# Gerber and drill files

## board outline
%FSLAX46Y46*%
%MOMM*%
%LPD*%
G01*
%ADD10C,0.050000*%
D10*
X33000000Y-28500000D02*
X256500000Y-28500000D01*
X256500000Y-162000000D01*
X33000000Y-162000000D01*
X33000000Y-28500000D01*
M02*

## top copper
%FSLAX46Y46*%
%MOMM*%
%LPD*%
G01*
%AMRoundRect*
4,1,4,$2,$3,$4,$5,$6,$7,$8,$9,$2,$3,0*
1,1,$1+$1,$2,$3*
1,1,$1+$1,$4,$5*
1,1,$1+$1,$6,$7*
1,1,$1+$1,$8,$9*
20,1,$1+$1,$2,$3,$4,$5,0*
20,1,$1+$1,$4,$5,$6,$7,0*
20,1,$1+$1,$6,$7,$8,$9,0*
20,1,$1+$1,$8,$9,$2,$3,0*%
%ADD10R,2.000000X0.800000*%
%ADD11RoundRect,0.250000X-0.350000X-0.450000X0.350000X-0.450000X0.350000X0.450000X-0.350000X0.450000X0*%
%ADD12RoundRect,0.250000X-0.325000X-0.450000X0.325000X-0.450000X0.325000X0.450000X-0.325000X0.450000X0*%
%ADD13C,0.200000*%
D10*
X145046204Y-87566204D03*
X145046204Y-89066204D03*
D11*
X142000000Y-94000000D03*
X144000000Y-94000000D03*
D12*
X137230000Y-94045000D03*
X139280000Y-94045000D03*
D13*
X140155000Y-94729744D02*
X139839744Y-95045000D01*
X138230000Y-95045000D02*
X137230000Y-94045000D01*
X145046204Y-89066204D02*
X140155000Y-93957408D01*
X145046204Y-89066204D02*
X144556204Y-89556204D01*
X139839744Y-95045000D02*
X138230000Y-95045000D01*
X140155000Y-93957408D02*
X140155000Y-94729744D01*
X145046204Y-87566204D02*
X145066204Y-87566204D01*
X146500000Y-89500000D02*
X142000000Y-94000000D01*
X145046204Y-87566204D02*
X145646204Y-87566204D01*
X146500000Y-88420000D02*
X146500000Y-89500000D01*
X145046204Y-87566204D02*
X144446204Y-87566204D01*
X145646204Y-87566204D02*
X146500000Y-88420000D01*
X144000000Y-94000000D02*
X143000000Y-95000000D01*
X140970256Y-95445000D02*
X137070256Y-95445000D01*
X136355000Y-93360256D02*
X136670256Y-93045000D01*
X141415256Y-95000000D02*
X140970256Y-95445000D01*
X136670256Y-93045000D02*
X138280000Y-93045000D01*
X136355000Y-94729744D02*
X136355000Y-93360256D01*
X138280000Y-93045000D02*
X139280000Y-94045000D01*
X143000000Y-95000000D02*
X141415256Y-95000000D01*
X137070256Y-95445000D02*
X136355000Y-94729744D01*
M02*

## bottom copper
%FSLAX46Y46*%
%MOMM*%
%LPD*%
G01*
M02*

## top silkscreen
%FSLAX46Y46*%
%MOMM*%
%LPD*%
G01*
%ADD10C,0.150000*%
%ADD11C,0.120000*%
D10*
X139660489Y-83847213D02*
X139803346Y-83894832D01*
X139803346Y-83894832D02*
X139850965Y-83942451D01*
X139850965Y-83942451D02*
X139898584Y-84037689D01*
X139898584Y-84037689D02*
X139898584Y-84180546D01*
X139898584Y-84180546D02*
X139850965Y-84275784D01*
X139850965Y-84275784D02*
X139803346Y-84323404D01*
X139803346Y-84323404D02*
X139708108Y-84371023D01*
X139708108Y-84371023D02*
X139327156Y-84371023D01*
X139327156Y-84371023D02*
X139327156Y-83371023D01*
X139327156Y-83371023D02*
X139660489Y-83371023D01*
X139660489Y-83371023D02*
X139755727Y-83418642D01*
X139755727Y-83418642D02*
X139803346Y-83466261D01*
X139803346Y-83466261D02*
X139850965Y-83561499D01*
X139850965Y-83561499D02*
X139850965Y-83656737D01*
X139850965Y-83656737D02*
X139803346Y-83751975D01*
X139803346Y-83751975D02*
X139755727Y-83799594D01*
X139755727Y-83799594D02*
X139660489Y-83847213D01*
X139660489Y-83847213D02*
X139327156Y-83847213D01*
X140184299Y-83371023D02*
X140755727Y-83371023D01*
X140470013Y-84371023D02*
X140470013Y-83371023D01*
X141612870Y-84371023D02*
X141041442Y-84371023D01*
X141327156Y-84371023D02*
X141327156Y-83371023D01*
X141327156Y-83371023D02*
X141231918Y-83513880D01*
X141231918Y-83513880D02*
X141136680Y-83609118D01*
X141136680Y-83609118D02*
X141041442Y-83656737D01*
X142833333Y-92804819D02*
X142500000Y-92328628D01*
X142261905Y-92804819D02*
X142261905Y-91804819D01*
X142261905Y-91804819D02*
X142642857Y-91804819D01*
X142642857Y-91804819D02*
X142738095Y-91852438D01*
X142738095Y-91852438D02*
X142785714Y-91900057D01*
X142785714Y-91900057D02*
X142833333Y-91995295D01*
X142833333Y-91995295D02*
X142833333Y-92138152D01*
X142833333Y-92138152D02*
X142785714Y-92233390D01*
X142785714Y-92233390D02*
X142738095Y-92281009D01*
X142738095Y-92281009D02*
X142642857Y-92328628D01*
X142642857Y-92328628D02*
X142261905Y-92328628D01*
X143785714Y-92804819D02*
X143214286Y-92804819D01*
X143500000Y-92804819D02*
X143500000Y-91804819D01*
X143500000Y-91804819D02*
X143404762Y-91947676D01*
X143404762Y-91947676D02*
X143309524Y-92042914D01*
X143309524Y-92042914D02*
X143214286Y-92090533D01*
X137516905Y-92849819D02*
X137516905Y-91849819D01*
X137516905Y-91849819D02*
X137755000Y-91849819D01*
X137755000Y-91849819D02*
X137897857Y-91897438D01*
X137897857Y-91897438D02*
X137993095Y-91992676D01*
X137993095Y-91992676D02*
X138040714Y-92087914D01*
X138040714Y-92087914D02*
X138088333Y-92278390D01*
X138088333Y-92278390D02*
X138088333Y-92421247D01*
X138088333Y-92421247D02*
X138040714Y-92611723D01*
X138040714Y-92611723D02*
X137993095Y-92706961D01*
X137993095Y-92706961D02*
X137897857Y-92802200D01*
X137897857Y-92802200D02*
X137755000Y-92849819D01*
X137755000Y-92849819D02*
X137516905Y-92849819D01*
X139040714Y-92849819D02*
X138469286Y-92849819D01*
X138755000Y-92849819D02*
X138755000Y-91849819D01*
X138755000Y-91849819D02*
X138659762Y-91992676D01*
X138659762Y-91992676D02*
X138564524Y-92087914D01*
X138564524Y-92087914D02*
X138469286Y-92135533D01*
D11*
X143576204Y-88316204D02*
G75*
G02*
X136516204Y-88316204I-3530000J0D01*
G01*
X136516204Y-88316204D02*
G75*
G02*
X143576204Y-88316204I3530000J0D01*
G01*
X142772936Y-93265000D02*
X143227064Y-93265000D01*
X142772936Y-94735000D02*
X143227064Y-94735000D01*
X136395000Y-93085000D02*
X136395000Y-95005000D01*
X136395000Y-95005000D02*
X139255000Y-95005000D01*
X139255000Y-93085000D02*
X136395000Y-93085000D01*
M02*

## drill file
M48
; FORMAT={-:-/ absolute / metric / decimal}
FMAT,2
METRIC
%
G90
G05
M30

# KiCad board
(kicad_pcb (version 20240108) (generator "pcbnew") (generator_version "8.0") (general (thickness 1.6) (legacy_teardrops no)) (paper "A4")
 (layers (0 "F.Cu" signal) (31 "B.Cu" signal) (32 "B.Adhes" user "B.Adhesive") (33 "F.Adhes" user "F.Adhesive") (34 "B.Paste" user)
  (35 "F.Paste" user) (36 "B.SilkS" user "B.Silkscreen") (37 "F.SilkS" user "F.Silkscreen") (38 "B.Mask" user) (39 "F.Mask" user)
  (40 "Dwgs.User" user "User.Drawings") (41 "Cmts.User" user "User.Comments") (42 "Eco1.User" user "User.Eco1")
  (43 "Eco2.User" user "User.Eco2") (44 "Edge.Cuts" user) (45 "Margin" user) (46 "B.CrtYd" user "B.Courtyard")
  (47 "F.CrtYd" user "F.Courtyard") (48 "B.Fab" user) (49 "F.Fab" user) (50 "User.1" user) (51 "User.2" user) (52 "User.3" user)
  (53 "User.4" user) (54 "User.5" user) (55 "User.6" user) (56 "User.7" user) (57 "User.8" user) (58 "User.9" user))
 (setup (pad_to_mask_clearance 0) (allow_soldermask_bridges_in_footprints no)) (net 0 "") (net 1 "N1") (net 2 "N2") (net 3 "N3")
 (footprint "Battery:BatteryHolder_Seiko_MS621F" (layer "F.Cu") (at 145.046204 88.316204)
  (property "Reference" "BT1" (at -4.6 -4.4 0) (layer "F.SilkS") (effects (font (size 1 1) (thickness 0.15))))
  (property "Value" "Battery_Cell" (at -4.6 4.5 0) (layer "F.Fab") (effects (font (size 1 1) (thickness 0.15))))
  (fp_circle (center -5 0) (end -1.47 0) (stroke (width 0.12) (type solid)) (fill none) (layer "F.SilkS"))
  (pad "1" smd rect (at 0 -0.75) (size 2 0.8) (layers "F.Cu" "F.Paste" "F.Mask") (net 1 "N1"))
  (pad "2" smd rect (at 0 0.75) (size 2 0.8) (layers "F.Cu" "F.Paste" "F.Mask") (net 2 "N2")))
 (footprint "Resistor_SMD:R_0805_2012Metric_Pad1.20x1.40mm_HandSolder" (layer "F.Cu") (at 143 94)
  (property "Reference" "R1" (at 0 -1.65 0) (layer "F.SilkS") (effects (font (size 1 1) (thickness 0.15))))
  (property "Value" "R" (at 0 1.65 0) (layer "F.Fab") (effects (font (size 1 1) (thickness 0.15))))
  (fp_line (start -0.227064 -0.735) (end 0.227064 -0.735) (stroke (width 0.12) (type solid)) (layer "F.SilkS"))
  (fp_line (start -0.227064 0.735) (end 0.227064 0.735) (stroke (width 0.12) (type solid)) (layer "F.SilkS"))
  (pad "1" smd roundrect (at -1 0) (size 1.2 1.4) (layers "F.Cu" "F.Paste" "F.Mask") (roundrect_rratio 0.208333) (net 1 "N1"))
  (pad "2" smd roundrect (at 1 0) (size 1.2 1.4) (layers "F.Cu" "F.Paste" "F.Mask") (roundrect_rratio 0.208333) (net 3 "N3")))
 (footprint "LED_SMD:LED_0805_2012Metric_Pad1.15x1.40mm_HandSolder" (layer "F.Cu") (at 138.255 94.045)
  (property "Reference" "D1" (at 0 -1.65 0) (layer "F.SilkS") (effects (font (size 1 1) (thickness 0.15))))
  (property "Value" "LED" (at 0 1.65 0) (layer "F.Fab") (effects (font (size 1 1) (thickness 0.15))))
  (fp_line (start -1.86 -0.96) (end -1.86 0.96) (stroke (width 0.12) (type solid)) (layer "F.SilkS"))
  (fp_line (start -1.86 0.96) (end 1 0.96) (stroke (width 0.12) (type solid)) (layer "F.SilkS"))
  (fp_line (start 1 -0.96) (end -1.86 -0.96) (stroke (width 0.12) (type solid)) (layer "F.SilkS"))
  (pad "1" smd roundrect (at -1.025 0) (size 1.15 1.4) (layers "F.Cu" "F.Paste" "F.Mask") (roundrect_rratio 0.217391) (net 2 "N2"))
  (pad "2" smd roundrect (at 1.025 0) (size 1.15 1.4) (layers "F.Cu" "F.Paste" "F.Mask") (roundrect_rratio 0.217391) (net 3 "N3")))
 (gr_rect (start 33 28.5) (end 256.5 162) (stroke (width 0.05) (type default)) (fill none) (layer "Edge.Cuts"))
 (segment (start 140.155 94.729744) (end 139.839744 95.045) (width 0.2) (layer "F.Cu") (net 2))
 (segment (start 138.23 95.045) (end 137.23 94.045) (width 0.2) (layer "F.Cu") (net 2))
 (segment (start 145.046204 89.066204) (end 140.155 93.957408) (width 0.2) (layer "F.Cu") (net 2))
 (segment (start 145.046204 89.066204) (end 144.556204 89.556204) (width 0.2) (layer "F.Cu") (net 2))
 (segment (start 139.839744 95.045) (end 138.23 95.045) (width 0.2) (layer "F.Cu") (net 2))
 (segment (start 140.155 93.957408) (end 140.155 94.729744) (width 0.2) (layer "F.Cu") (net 2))
 (segment (start 145.046204 87.566204) (end 145.066204 87.566204) (width 0.2) (layer "F.Cu") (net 1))
 (segment (start 146.5 89.5) (end 142 94) (width 0.2) (layer "F.Cu") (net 1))
 (segment (start 145.046204 87.566204) (end 145.646204 87.566204) (width 0.2) (layer "F.Cu") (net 1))
 (segment (start 146.5 88.42) (end 146.5 89.5) (width 0.2) (layer "F.Cu") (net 1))
 (segment (start 145.046204 87.566204) (end 144.446204 87.566204) (width 0.2) (layer "F.Cu") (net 1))
 (segment (start 145.646204 87.566204) (end 146.5 88.42) (width 0.2) (layer "F.Cu") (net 1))
 (segment (start 144 94) (end 143 95) (width 0.2) (layer "F.Cu") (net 3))
 (segment (start 140.970256 95.445) (end 137.070256 95.445) (width 0.2) (layer "F.Cu") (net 3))
 (segment (start 136.355 93.360256) (end 136.670256 93.045) (width 0.2) (layer "F.Cu") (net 3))
 (segment (start 141.415256 95) (end 140.970256 95.445) (width 0.2) (layer "F.Cu") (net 3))
 (segment (start 136.670256 93.045) (end 138.28 93.045) (width 0.2) (layer "F.Cu") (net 3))
 (segment (start 136.355 94.729744) (end 136.355 93.360256) (width 0.2) (layer "F.Cu") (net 3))
 (segment (start 138.28 93.045) (end 139.28 94.045) (width 0.2) (layer "F.Cu") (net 3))
 (segment (start 143 95) (end 141.415256 95) (width 0.2) (layer "F.Cu") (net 3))
 (segment (start 137.070256 95.445) (end 136.355 94.729744) (width 0.2) (layer "F.Cu") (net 3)))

